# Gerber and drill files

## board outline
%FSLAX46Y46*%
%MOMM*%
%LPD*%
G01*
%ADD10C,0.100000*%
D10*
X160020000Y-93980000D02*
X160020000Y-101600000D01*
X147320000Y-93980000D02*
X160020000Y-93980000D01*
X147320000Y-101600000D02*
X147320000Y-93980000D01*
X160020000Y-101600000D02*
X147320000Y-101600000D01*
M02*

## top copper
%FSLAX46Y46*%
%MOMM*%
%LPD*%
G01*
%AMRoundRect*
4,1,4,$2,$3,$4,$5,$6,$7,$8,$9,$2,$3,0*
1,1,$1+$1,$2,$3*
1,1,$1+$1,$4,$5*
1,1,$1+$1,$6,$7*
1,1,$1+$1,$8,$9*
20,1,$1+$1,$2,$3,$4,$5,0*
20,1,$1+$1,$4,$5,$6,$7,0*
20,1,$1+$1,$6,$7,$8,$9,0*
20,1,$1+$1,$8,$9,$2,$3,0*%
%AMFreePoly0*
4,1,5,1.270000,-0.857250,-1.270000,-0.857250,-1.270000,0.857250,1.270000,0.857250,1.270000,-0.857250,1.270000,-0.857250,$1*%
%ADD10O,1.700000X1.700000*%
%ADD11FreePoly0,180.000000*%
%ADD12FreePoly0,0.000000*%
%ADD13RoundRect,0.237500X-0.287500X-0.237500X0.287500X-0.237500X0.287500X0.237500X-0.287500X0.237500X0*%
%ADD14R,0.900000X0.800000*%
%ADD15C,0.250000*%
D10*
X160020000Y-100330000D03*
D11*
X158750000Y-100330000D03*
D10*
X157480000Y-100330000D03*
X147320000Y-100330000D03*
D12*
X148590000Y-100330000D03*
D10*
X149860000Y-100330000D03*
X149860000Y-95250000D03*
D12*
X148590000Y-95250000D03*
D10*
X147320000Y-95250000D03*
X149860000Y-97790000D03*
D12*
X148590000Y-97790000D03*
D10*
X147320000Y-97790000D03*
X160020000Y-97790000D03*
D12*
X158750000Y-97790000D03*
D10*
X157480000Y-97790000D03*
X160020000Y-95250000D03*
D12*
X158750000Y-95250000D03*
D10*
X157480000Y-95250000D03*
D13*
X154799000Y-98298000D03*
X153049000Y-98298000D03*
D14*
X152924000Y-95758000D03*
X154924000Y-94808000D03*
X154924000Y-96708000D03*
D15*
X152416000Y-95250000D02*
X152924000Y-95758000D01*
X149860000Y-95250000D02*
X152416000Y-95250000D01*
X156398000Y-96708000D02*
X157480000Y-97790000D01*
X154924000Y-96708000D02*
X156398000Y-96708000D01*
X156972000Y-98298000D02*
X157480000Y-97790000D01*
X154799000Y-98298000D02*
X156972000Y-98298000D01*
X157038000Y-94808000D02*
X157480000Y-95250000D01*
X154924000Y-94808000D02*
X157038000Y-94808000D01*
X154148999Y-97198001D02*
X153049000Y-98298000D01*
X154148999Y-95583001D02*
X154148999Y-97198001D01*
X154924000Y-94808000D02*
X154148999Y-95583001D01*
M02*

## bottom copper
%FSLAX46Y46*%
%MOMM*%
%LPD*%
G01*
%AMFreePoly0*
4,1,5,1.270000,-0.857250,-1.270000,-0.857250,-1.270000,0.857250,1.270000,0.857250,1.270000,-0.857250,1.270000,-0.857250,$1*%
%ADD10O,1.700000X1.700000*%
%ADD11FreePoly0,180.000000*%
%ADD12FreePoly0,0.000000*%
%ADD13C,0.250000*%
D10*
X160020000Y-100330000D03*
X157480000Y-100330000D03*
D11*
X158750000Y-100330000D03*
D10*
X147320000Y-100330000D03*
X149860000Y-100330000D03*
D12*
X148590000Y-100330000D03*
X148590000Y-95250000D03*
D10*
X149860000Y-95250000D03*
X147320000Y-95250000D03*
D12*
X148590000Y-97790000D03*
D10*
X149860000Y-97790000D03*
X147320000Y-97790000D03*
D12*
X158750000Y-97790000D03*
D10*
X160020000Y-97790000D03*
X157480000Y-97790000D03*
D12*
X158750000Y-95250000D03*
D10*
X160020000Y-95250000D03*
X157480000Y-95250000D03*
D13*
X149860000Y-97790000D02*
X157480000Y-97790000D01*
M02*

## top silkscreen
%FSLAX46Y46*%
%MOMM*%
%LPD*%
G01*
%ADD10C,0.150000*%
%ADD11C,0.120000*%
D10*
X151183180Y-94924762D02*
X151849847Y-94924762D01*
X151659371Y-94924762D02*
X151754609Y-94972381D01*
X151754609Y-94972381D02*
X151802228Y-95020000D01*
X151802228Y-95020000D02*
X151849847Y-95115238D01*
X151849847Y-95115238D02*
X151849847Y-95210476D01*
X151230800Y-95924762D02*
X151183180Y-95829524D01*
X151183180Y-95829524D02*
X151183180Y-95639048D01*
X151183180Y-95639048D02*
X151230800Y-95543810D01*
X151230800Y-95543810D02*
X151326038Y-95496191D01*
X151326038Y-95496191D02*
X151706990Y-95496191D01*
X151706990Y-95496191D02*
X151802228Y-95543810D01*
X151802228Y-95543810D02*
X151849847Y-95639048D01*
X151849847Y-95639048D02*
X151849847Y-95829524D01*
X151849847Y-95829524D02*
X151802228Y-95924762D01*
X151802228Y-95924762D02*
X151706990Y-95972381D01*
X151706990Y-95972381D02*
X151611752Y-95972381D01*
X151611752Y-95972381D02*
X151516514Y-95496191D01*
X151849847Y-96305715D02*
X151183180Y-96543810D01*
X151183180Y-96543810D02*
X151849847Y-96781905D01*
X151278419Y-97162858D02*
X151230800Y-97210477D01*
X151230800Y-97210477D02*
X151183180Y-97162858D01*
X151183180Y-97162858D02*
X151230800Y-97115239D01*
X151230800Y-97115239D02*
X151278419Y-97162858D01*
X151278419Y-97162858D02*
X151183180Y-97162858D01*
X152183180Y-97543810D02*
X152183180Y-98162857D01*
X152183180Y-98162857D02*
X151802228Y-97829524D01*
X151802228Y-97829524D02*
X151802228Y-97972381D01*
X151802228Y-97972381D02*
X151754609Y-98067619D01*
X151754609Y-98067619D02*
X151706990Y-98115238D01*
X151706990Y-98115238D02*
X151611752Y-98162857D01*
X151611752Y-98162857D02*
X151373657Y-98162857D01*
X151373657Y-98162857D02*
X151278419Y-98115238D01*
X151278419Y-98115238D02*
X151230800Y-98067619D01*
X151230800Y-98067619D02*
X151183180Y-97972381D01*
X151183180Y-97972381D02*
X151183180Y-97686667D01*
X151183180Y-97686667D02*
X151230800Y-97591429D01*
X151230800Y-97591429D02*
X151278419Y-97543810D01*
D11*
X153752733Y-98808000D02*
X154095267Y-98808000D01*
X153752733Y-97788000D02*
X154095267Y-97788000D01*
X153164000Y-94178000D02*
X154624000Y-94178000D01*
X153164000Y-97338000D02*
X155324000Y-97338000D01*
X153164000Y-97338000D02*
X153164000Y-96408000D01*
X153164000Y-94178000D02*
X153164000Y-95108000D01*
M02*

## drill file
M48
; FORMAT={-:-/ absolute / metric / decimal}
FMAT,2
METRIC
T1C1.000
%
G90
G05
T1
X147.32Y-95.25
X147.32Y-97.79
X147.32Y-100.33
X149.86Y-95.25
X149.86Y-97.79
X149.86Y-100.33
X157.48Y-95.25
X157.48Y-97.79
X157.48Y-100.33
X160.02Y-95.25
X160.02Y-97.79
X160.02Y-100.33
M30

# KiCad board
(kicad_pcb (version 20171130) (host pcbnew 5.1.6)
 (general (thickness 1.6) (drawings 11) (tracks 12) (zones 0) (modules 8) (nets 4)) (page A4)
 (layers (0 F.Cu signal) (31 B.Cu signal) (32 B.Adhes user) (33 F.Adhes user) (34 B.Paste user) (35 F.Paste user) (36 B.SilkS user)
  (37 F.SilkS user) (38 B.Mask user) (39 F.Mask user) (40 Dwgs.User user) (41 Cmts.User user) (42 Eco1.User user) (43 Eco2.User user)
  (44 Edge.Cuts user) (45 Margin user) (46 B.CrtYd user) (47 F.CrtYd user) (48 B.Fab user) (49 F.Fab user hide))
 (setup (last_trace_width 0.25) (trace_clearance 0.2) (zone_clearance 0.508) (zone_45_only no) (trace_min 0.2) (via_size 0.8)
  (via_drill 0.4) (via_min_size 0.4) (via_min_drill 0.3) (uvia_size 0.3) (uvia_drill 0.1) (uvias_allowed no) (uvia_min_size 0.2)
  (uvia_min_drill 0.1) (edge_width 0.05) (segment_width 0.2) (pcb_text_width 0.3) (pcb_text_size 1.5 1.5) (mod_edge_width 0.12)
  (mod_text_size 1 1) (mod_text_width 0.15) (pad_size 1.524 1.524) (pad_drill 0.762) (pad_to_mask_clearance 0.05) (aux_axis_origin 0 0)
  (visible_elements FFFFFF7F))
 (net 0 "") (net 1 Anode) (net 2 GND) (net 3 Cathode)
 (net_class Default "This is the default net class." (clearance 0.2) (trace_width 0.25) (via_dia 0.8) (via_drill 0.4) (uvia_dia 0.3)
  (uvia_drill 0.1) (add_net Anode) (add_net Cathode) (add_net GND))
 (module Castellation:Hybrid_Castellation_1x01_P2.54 (layer F.Cu) (at 158.75 100.33 180)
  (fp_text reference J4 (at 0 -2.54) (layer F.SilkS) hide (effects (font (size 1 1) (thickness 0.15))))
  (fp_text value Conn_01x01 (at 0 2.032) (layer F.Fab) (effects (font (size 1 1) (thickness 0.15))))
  (pad 1 thru_hole oval (at -1.27 0 180) (size 1.7 1.7) (drill 1) (layers *.Cu *.Mask))
  (pad 1 connect custom (at 0 0 180) (size 2.54 1.7145) (layers F.Cu F.Mask) (zone_connect 0) (options (clearance outline) (anchor rect))
   (primitives))
  (pad 1 thru_hole oval (at 1.27 0 180) (size 1.7 1.7) (drill 1) (layers *.Cu *.Mask))
  (pad 1 connect custom (at 0 0 180) (size 2.54 1.7145) (layers B.Cu B.Mask) (zone_connect 0) (options (clearance outline) (anchor rect))
   (primitives)))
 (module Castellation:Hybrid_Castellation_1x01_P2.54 (layer F.Cu) (at 148.59 100.33)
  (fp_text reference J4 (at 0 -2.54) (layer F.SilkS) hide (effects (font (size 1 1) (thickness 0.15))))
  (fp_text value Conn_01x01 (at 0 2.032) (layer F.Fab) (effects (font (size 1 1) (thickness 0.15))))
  (pad 1 thru_hole oval (at -1.27 0) (size 1.7 1.7) (drill 1) (layers *.Cu *.Mask))
  (pad 1 connect custom (at 0 0) (size 2.54 1.7145) (layers F.Cu F.Mask) (zone_connect 0) (options (clearance outline) (anchor rect))
   (primitives))
  (pad 1 thru_hole oval (at 1.27 0) (size 1.7 1.7) (drill 1) (layers *.Cu *.Mask))
  (pad 1 connect custom (at 0 0) (size 2.54 1.7145) (layers B.Cu B.Mask) (zone_connect 0) (options (clearance outline) (anchor rect))
   (primitives)))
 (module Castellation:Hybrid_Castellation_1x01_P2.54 (layer F.Cu) (at 148.59 95.25)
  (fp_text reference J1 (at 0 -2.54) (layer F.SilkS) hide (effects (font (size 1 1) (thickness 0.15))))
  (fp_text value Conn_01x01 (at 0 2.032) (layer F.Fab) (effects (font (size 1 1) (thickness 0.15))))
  (pad 1 connect custom (at 0 0) (size 2.54 1.7145) (layers B.Cu B.Mask) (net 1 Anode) (zone_connect 0)
   (options (clearance outline) (anchor rect)) (primitives))
  (pad 1 thru_hole oval (at 1.27 0) (size 1.7 1.7) (drill 1) (layers *.Cu *.Mask) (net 1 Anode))
  (pad 1 connect custom (at 0 0) (size 2.54 1.7145) (layers F.Cu F.Mask) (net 1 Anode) (zone_connect 0)
   (options (clearance outline) (anchor rect)) (primitives))
  (pad 1 thru_hole oval (at -1.27 0) (size 1.7 1.7) (drill 1) (layers *.Cu *.Mask) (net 1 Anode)))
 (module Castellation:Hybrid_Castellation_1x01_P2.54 (layer F.Cu) (at 148.59 97.79)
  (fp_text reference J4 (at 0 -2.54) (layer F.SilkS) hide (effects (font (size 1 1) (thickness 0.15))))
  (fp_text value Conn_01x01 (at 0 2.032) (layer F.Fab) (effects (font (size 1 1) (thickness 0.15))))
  (pad 1 connect custom (at 0 0) (size 2.54 1.7145) (layers B.Cu B.Mask) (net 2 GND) (zone_connect 0)
   (options (clearance outline) (anchor rect)) (primitives))
  (pad 1 thru_hole oval (at 1.27 0) (size 1.7 1.7) (drill 1) (layers *.Cu *.Mask) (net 2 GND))
  (pad 1 connect custom (at 0 0) (size 2.54 1.7145) (layers F.Cu F.Mask) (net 2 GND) (zone_connect 0)
   (options (clearance outline) (anchor rect)) (primitives))
  (pad 1 thru_hole oval (at -1.27 0) (size 1.7 1.7) (drill 1) (layers *.Cu *.Mask) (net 2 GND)))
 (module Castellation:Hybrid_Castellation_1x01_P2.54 (layer F.Cu) (at 158.75 97.79)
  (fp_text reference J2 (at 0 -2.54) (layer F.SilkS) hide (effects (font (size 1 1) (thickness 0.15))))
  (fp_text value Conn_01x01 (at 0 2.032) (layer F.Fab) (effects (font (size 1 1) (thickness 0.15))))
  (pad 1 connect custom (at 0 0) (size 2.54 1.7145) (layers B.Cu B.Mask) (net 2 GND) (zone_connect 0)
   (options (clearance outline) (anchor rect)) (primitives))
  (pad 1 thru_hole oval (at 1.27 0) (size 1.7 1.7) (drill 1) (layers *.Cu *.Mask) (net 2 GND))
  (pad 1 connect custom (at 0 0) (size 2.54 1.7145) (layers F.Cu F.Mask) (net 2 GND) (zone_connect 0)
   (options (clearance outline) (anchor rect)) (primitives))
  (pad 1 thru_hole oval (at -1.27 0) (size 1.7 1.7) (drill 1) (layers *.Cu *.Mask) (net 2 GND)))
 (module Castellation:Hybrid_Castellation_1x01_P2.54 (layer F.Cu) (at 158.75 95.25)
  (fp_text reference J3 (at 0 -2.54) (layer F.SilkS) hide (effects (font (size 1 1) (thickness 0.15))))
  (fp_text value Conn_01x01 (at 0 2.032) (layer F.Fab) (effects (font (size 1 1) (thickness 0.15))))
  (pad 1 connect custom (at 0 0) (size 2.54 1.7145) (layers B.Cu B.Mask) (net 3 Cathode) (zone_connect 0)
   (options (clearance outline) (anchor rect)) (primitives))
  (pad 1 thru_hole oval (at 1.27 0) (size 1.7 1.7) (drill 1) (layers *.Cu *.Mask) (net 3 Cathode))
  (pad 1 connect custom (at 0 0) (size 2.54 1.7145) (layers F.Cu F.Mask) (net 3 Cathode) (zone_connect 0)
   (options (clearance outline) (anchor rect)) (primitives))
  (pad 1 thru_hole oval (at -1.27 0) (size 1.7 1.7) (drill 1) (layers *.Cu *.Mask) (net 3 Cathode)))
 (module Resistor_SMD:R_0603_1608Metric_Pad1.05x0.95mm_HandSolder (layer F.Cu) (at 153.924 98.298)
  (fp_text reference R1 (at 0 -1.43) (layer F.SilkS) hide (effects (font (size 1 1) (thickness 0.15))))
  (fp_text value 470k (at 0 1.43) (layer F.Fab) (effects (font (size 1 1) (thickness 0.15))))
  (fp_line (start -0.171267 0.51) (end 0.171267 0.51) (layer F.SilkS) (width 0.12))
  (fp_line (start -0.171267 -0.51) (end 0.171267 -0.51) (layer F.SilkS) (width 0.12))
  (pad 2 smd roundrect (at 0.875 0) (size 1.05 0.95) (layers F.Cu F.Paste F.Mask) (roundrect_rratio 0.25) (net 2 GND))
  (pad 1 smd roundrect (at -0.875 0) (size 1.05 0.95) (layers F.Cu F.Paste F.Mask) (roundrect_rratio 0.25) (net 3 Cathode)))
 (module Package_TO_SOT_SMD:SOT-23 (layer F.Cu) (at 153.924 95.758 180)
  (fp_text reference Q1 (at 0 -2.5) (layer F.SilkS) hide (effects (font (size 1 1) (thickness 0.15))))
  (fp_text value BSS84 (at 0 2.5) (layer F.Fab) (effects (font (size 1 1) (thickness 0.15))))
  (fp_line (start 0.76 1.58) (end -0.7 1.58) (layer F.SilkS) (width 0.12))
  (fp_line (start 0.76 -1.58) (end -1.4 -1.58) (layer F.SilkS) (width 0.12))
  (fp_line (start 0.76 -1.58) (end 0.76 -0.65) (layer F.SilkS) (width 0.12))
  (fp_line (start 0.76 1.58) (end 0.76 0.65) (layer F.SilkS) (width 0.12))
  (pad 3 smd rect (at 1 0 180) (size 0.9 0.8) (layers F.Cu F.Paste F.Mask) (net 1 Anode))
  (pad 2 smd rect (at -1 0.95 180) (size 0.9 0.8) (layers F.Cu F.Paste F.Mask) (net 3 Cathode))
  (pad 1 smd rect (at -1 -0.95 180) (size 0.9 0.8) (layers F.Cu F.Paste F.Mask) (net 2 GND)))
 (gr_line (start 160.02 93.98) (end 160.02 101.6) (layer Edge.Cuts) (width 0.1))
 (gr_line (start 147.32 93.98) (end 160.02 93.98) (layer Edge.Cuts) (width 0.1))
 (gr_line (start 147.32 101.6) (end 147.32 93.98) (layer Edge.Cuts) (width 0.1))
 (gr_line (start 160.02 101.6) (end 147.32 101.6) (layer Edge.Cuts) (width 0.1))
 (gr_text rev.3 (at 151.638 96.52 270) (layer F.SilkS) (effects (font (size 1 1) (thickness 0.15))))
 (segment (start 152.416 95.25) (end 152.924 95.758) (width 0.25) (layer F.Cu) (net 1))
 (segment (start 149.86 95.25) (end 152.416 95.25) (width 0.25) (layer F.Cu) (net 1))
 (segment (start 156.398 96.708) (end 157.48 97.79) (width 0.25) (layer F.Cu) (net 2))
 (segment (start 154.924 96.708) (end 156.398 96.708) (width 0.25) (layer F.Cu) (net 2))
 (segment (start 156.972 98.298) (end 157.48 97.79) (width 0.25) (layer F.Cu) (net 2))
 (segment (start 154.799 98.298) (end 156.972 98.298) (width 0.25) (layer F.Cu) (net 2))
 (segment (start 149.86 97.79) (end 157.48 97.79) (width 0.25) (layer B.Cu) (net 2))
 (segment (start 157.038 94.808) (end 157.48 95.25) (width 0.25) (layer F.Cu) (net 3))
 (segment (start 154.924 94.808) (end 157.038 94.808) (width 0.25) (layer F.Cu) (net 3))
 (segment (start 154.148999 97.198001) (end 153.049 98.298) (width 0.25) (layer F.Cu) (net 3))
 (segment (start 154.148999 95.583001) (end 154.148999 97.198001) (width 0.25) (layer F.Cu) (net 3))
 (segment (start 154.924 94.808) (end 154.148999 95.583001) (width 0.25) (layer F.Cu) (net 3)))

